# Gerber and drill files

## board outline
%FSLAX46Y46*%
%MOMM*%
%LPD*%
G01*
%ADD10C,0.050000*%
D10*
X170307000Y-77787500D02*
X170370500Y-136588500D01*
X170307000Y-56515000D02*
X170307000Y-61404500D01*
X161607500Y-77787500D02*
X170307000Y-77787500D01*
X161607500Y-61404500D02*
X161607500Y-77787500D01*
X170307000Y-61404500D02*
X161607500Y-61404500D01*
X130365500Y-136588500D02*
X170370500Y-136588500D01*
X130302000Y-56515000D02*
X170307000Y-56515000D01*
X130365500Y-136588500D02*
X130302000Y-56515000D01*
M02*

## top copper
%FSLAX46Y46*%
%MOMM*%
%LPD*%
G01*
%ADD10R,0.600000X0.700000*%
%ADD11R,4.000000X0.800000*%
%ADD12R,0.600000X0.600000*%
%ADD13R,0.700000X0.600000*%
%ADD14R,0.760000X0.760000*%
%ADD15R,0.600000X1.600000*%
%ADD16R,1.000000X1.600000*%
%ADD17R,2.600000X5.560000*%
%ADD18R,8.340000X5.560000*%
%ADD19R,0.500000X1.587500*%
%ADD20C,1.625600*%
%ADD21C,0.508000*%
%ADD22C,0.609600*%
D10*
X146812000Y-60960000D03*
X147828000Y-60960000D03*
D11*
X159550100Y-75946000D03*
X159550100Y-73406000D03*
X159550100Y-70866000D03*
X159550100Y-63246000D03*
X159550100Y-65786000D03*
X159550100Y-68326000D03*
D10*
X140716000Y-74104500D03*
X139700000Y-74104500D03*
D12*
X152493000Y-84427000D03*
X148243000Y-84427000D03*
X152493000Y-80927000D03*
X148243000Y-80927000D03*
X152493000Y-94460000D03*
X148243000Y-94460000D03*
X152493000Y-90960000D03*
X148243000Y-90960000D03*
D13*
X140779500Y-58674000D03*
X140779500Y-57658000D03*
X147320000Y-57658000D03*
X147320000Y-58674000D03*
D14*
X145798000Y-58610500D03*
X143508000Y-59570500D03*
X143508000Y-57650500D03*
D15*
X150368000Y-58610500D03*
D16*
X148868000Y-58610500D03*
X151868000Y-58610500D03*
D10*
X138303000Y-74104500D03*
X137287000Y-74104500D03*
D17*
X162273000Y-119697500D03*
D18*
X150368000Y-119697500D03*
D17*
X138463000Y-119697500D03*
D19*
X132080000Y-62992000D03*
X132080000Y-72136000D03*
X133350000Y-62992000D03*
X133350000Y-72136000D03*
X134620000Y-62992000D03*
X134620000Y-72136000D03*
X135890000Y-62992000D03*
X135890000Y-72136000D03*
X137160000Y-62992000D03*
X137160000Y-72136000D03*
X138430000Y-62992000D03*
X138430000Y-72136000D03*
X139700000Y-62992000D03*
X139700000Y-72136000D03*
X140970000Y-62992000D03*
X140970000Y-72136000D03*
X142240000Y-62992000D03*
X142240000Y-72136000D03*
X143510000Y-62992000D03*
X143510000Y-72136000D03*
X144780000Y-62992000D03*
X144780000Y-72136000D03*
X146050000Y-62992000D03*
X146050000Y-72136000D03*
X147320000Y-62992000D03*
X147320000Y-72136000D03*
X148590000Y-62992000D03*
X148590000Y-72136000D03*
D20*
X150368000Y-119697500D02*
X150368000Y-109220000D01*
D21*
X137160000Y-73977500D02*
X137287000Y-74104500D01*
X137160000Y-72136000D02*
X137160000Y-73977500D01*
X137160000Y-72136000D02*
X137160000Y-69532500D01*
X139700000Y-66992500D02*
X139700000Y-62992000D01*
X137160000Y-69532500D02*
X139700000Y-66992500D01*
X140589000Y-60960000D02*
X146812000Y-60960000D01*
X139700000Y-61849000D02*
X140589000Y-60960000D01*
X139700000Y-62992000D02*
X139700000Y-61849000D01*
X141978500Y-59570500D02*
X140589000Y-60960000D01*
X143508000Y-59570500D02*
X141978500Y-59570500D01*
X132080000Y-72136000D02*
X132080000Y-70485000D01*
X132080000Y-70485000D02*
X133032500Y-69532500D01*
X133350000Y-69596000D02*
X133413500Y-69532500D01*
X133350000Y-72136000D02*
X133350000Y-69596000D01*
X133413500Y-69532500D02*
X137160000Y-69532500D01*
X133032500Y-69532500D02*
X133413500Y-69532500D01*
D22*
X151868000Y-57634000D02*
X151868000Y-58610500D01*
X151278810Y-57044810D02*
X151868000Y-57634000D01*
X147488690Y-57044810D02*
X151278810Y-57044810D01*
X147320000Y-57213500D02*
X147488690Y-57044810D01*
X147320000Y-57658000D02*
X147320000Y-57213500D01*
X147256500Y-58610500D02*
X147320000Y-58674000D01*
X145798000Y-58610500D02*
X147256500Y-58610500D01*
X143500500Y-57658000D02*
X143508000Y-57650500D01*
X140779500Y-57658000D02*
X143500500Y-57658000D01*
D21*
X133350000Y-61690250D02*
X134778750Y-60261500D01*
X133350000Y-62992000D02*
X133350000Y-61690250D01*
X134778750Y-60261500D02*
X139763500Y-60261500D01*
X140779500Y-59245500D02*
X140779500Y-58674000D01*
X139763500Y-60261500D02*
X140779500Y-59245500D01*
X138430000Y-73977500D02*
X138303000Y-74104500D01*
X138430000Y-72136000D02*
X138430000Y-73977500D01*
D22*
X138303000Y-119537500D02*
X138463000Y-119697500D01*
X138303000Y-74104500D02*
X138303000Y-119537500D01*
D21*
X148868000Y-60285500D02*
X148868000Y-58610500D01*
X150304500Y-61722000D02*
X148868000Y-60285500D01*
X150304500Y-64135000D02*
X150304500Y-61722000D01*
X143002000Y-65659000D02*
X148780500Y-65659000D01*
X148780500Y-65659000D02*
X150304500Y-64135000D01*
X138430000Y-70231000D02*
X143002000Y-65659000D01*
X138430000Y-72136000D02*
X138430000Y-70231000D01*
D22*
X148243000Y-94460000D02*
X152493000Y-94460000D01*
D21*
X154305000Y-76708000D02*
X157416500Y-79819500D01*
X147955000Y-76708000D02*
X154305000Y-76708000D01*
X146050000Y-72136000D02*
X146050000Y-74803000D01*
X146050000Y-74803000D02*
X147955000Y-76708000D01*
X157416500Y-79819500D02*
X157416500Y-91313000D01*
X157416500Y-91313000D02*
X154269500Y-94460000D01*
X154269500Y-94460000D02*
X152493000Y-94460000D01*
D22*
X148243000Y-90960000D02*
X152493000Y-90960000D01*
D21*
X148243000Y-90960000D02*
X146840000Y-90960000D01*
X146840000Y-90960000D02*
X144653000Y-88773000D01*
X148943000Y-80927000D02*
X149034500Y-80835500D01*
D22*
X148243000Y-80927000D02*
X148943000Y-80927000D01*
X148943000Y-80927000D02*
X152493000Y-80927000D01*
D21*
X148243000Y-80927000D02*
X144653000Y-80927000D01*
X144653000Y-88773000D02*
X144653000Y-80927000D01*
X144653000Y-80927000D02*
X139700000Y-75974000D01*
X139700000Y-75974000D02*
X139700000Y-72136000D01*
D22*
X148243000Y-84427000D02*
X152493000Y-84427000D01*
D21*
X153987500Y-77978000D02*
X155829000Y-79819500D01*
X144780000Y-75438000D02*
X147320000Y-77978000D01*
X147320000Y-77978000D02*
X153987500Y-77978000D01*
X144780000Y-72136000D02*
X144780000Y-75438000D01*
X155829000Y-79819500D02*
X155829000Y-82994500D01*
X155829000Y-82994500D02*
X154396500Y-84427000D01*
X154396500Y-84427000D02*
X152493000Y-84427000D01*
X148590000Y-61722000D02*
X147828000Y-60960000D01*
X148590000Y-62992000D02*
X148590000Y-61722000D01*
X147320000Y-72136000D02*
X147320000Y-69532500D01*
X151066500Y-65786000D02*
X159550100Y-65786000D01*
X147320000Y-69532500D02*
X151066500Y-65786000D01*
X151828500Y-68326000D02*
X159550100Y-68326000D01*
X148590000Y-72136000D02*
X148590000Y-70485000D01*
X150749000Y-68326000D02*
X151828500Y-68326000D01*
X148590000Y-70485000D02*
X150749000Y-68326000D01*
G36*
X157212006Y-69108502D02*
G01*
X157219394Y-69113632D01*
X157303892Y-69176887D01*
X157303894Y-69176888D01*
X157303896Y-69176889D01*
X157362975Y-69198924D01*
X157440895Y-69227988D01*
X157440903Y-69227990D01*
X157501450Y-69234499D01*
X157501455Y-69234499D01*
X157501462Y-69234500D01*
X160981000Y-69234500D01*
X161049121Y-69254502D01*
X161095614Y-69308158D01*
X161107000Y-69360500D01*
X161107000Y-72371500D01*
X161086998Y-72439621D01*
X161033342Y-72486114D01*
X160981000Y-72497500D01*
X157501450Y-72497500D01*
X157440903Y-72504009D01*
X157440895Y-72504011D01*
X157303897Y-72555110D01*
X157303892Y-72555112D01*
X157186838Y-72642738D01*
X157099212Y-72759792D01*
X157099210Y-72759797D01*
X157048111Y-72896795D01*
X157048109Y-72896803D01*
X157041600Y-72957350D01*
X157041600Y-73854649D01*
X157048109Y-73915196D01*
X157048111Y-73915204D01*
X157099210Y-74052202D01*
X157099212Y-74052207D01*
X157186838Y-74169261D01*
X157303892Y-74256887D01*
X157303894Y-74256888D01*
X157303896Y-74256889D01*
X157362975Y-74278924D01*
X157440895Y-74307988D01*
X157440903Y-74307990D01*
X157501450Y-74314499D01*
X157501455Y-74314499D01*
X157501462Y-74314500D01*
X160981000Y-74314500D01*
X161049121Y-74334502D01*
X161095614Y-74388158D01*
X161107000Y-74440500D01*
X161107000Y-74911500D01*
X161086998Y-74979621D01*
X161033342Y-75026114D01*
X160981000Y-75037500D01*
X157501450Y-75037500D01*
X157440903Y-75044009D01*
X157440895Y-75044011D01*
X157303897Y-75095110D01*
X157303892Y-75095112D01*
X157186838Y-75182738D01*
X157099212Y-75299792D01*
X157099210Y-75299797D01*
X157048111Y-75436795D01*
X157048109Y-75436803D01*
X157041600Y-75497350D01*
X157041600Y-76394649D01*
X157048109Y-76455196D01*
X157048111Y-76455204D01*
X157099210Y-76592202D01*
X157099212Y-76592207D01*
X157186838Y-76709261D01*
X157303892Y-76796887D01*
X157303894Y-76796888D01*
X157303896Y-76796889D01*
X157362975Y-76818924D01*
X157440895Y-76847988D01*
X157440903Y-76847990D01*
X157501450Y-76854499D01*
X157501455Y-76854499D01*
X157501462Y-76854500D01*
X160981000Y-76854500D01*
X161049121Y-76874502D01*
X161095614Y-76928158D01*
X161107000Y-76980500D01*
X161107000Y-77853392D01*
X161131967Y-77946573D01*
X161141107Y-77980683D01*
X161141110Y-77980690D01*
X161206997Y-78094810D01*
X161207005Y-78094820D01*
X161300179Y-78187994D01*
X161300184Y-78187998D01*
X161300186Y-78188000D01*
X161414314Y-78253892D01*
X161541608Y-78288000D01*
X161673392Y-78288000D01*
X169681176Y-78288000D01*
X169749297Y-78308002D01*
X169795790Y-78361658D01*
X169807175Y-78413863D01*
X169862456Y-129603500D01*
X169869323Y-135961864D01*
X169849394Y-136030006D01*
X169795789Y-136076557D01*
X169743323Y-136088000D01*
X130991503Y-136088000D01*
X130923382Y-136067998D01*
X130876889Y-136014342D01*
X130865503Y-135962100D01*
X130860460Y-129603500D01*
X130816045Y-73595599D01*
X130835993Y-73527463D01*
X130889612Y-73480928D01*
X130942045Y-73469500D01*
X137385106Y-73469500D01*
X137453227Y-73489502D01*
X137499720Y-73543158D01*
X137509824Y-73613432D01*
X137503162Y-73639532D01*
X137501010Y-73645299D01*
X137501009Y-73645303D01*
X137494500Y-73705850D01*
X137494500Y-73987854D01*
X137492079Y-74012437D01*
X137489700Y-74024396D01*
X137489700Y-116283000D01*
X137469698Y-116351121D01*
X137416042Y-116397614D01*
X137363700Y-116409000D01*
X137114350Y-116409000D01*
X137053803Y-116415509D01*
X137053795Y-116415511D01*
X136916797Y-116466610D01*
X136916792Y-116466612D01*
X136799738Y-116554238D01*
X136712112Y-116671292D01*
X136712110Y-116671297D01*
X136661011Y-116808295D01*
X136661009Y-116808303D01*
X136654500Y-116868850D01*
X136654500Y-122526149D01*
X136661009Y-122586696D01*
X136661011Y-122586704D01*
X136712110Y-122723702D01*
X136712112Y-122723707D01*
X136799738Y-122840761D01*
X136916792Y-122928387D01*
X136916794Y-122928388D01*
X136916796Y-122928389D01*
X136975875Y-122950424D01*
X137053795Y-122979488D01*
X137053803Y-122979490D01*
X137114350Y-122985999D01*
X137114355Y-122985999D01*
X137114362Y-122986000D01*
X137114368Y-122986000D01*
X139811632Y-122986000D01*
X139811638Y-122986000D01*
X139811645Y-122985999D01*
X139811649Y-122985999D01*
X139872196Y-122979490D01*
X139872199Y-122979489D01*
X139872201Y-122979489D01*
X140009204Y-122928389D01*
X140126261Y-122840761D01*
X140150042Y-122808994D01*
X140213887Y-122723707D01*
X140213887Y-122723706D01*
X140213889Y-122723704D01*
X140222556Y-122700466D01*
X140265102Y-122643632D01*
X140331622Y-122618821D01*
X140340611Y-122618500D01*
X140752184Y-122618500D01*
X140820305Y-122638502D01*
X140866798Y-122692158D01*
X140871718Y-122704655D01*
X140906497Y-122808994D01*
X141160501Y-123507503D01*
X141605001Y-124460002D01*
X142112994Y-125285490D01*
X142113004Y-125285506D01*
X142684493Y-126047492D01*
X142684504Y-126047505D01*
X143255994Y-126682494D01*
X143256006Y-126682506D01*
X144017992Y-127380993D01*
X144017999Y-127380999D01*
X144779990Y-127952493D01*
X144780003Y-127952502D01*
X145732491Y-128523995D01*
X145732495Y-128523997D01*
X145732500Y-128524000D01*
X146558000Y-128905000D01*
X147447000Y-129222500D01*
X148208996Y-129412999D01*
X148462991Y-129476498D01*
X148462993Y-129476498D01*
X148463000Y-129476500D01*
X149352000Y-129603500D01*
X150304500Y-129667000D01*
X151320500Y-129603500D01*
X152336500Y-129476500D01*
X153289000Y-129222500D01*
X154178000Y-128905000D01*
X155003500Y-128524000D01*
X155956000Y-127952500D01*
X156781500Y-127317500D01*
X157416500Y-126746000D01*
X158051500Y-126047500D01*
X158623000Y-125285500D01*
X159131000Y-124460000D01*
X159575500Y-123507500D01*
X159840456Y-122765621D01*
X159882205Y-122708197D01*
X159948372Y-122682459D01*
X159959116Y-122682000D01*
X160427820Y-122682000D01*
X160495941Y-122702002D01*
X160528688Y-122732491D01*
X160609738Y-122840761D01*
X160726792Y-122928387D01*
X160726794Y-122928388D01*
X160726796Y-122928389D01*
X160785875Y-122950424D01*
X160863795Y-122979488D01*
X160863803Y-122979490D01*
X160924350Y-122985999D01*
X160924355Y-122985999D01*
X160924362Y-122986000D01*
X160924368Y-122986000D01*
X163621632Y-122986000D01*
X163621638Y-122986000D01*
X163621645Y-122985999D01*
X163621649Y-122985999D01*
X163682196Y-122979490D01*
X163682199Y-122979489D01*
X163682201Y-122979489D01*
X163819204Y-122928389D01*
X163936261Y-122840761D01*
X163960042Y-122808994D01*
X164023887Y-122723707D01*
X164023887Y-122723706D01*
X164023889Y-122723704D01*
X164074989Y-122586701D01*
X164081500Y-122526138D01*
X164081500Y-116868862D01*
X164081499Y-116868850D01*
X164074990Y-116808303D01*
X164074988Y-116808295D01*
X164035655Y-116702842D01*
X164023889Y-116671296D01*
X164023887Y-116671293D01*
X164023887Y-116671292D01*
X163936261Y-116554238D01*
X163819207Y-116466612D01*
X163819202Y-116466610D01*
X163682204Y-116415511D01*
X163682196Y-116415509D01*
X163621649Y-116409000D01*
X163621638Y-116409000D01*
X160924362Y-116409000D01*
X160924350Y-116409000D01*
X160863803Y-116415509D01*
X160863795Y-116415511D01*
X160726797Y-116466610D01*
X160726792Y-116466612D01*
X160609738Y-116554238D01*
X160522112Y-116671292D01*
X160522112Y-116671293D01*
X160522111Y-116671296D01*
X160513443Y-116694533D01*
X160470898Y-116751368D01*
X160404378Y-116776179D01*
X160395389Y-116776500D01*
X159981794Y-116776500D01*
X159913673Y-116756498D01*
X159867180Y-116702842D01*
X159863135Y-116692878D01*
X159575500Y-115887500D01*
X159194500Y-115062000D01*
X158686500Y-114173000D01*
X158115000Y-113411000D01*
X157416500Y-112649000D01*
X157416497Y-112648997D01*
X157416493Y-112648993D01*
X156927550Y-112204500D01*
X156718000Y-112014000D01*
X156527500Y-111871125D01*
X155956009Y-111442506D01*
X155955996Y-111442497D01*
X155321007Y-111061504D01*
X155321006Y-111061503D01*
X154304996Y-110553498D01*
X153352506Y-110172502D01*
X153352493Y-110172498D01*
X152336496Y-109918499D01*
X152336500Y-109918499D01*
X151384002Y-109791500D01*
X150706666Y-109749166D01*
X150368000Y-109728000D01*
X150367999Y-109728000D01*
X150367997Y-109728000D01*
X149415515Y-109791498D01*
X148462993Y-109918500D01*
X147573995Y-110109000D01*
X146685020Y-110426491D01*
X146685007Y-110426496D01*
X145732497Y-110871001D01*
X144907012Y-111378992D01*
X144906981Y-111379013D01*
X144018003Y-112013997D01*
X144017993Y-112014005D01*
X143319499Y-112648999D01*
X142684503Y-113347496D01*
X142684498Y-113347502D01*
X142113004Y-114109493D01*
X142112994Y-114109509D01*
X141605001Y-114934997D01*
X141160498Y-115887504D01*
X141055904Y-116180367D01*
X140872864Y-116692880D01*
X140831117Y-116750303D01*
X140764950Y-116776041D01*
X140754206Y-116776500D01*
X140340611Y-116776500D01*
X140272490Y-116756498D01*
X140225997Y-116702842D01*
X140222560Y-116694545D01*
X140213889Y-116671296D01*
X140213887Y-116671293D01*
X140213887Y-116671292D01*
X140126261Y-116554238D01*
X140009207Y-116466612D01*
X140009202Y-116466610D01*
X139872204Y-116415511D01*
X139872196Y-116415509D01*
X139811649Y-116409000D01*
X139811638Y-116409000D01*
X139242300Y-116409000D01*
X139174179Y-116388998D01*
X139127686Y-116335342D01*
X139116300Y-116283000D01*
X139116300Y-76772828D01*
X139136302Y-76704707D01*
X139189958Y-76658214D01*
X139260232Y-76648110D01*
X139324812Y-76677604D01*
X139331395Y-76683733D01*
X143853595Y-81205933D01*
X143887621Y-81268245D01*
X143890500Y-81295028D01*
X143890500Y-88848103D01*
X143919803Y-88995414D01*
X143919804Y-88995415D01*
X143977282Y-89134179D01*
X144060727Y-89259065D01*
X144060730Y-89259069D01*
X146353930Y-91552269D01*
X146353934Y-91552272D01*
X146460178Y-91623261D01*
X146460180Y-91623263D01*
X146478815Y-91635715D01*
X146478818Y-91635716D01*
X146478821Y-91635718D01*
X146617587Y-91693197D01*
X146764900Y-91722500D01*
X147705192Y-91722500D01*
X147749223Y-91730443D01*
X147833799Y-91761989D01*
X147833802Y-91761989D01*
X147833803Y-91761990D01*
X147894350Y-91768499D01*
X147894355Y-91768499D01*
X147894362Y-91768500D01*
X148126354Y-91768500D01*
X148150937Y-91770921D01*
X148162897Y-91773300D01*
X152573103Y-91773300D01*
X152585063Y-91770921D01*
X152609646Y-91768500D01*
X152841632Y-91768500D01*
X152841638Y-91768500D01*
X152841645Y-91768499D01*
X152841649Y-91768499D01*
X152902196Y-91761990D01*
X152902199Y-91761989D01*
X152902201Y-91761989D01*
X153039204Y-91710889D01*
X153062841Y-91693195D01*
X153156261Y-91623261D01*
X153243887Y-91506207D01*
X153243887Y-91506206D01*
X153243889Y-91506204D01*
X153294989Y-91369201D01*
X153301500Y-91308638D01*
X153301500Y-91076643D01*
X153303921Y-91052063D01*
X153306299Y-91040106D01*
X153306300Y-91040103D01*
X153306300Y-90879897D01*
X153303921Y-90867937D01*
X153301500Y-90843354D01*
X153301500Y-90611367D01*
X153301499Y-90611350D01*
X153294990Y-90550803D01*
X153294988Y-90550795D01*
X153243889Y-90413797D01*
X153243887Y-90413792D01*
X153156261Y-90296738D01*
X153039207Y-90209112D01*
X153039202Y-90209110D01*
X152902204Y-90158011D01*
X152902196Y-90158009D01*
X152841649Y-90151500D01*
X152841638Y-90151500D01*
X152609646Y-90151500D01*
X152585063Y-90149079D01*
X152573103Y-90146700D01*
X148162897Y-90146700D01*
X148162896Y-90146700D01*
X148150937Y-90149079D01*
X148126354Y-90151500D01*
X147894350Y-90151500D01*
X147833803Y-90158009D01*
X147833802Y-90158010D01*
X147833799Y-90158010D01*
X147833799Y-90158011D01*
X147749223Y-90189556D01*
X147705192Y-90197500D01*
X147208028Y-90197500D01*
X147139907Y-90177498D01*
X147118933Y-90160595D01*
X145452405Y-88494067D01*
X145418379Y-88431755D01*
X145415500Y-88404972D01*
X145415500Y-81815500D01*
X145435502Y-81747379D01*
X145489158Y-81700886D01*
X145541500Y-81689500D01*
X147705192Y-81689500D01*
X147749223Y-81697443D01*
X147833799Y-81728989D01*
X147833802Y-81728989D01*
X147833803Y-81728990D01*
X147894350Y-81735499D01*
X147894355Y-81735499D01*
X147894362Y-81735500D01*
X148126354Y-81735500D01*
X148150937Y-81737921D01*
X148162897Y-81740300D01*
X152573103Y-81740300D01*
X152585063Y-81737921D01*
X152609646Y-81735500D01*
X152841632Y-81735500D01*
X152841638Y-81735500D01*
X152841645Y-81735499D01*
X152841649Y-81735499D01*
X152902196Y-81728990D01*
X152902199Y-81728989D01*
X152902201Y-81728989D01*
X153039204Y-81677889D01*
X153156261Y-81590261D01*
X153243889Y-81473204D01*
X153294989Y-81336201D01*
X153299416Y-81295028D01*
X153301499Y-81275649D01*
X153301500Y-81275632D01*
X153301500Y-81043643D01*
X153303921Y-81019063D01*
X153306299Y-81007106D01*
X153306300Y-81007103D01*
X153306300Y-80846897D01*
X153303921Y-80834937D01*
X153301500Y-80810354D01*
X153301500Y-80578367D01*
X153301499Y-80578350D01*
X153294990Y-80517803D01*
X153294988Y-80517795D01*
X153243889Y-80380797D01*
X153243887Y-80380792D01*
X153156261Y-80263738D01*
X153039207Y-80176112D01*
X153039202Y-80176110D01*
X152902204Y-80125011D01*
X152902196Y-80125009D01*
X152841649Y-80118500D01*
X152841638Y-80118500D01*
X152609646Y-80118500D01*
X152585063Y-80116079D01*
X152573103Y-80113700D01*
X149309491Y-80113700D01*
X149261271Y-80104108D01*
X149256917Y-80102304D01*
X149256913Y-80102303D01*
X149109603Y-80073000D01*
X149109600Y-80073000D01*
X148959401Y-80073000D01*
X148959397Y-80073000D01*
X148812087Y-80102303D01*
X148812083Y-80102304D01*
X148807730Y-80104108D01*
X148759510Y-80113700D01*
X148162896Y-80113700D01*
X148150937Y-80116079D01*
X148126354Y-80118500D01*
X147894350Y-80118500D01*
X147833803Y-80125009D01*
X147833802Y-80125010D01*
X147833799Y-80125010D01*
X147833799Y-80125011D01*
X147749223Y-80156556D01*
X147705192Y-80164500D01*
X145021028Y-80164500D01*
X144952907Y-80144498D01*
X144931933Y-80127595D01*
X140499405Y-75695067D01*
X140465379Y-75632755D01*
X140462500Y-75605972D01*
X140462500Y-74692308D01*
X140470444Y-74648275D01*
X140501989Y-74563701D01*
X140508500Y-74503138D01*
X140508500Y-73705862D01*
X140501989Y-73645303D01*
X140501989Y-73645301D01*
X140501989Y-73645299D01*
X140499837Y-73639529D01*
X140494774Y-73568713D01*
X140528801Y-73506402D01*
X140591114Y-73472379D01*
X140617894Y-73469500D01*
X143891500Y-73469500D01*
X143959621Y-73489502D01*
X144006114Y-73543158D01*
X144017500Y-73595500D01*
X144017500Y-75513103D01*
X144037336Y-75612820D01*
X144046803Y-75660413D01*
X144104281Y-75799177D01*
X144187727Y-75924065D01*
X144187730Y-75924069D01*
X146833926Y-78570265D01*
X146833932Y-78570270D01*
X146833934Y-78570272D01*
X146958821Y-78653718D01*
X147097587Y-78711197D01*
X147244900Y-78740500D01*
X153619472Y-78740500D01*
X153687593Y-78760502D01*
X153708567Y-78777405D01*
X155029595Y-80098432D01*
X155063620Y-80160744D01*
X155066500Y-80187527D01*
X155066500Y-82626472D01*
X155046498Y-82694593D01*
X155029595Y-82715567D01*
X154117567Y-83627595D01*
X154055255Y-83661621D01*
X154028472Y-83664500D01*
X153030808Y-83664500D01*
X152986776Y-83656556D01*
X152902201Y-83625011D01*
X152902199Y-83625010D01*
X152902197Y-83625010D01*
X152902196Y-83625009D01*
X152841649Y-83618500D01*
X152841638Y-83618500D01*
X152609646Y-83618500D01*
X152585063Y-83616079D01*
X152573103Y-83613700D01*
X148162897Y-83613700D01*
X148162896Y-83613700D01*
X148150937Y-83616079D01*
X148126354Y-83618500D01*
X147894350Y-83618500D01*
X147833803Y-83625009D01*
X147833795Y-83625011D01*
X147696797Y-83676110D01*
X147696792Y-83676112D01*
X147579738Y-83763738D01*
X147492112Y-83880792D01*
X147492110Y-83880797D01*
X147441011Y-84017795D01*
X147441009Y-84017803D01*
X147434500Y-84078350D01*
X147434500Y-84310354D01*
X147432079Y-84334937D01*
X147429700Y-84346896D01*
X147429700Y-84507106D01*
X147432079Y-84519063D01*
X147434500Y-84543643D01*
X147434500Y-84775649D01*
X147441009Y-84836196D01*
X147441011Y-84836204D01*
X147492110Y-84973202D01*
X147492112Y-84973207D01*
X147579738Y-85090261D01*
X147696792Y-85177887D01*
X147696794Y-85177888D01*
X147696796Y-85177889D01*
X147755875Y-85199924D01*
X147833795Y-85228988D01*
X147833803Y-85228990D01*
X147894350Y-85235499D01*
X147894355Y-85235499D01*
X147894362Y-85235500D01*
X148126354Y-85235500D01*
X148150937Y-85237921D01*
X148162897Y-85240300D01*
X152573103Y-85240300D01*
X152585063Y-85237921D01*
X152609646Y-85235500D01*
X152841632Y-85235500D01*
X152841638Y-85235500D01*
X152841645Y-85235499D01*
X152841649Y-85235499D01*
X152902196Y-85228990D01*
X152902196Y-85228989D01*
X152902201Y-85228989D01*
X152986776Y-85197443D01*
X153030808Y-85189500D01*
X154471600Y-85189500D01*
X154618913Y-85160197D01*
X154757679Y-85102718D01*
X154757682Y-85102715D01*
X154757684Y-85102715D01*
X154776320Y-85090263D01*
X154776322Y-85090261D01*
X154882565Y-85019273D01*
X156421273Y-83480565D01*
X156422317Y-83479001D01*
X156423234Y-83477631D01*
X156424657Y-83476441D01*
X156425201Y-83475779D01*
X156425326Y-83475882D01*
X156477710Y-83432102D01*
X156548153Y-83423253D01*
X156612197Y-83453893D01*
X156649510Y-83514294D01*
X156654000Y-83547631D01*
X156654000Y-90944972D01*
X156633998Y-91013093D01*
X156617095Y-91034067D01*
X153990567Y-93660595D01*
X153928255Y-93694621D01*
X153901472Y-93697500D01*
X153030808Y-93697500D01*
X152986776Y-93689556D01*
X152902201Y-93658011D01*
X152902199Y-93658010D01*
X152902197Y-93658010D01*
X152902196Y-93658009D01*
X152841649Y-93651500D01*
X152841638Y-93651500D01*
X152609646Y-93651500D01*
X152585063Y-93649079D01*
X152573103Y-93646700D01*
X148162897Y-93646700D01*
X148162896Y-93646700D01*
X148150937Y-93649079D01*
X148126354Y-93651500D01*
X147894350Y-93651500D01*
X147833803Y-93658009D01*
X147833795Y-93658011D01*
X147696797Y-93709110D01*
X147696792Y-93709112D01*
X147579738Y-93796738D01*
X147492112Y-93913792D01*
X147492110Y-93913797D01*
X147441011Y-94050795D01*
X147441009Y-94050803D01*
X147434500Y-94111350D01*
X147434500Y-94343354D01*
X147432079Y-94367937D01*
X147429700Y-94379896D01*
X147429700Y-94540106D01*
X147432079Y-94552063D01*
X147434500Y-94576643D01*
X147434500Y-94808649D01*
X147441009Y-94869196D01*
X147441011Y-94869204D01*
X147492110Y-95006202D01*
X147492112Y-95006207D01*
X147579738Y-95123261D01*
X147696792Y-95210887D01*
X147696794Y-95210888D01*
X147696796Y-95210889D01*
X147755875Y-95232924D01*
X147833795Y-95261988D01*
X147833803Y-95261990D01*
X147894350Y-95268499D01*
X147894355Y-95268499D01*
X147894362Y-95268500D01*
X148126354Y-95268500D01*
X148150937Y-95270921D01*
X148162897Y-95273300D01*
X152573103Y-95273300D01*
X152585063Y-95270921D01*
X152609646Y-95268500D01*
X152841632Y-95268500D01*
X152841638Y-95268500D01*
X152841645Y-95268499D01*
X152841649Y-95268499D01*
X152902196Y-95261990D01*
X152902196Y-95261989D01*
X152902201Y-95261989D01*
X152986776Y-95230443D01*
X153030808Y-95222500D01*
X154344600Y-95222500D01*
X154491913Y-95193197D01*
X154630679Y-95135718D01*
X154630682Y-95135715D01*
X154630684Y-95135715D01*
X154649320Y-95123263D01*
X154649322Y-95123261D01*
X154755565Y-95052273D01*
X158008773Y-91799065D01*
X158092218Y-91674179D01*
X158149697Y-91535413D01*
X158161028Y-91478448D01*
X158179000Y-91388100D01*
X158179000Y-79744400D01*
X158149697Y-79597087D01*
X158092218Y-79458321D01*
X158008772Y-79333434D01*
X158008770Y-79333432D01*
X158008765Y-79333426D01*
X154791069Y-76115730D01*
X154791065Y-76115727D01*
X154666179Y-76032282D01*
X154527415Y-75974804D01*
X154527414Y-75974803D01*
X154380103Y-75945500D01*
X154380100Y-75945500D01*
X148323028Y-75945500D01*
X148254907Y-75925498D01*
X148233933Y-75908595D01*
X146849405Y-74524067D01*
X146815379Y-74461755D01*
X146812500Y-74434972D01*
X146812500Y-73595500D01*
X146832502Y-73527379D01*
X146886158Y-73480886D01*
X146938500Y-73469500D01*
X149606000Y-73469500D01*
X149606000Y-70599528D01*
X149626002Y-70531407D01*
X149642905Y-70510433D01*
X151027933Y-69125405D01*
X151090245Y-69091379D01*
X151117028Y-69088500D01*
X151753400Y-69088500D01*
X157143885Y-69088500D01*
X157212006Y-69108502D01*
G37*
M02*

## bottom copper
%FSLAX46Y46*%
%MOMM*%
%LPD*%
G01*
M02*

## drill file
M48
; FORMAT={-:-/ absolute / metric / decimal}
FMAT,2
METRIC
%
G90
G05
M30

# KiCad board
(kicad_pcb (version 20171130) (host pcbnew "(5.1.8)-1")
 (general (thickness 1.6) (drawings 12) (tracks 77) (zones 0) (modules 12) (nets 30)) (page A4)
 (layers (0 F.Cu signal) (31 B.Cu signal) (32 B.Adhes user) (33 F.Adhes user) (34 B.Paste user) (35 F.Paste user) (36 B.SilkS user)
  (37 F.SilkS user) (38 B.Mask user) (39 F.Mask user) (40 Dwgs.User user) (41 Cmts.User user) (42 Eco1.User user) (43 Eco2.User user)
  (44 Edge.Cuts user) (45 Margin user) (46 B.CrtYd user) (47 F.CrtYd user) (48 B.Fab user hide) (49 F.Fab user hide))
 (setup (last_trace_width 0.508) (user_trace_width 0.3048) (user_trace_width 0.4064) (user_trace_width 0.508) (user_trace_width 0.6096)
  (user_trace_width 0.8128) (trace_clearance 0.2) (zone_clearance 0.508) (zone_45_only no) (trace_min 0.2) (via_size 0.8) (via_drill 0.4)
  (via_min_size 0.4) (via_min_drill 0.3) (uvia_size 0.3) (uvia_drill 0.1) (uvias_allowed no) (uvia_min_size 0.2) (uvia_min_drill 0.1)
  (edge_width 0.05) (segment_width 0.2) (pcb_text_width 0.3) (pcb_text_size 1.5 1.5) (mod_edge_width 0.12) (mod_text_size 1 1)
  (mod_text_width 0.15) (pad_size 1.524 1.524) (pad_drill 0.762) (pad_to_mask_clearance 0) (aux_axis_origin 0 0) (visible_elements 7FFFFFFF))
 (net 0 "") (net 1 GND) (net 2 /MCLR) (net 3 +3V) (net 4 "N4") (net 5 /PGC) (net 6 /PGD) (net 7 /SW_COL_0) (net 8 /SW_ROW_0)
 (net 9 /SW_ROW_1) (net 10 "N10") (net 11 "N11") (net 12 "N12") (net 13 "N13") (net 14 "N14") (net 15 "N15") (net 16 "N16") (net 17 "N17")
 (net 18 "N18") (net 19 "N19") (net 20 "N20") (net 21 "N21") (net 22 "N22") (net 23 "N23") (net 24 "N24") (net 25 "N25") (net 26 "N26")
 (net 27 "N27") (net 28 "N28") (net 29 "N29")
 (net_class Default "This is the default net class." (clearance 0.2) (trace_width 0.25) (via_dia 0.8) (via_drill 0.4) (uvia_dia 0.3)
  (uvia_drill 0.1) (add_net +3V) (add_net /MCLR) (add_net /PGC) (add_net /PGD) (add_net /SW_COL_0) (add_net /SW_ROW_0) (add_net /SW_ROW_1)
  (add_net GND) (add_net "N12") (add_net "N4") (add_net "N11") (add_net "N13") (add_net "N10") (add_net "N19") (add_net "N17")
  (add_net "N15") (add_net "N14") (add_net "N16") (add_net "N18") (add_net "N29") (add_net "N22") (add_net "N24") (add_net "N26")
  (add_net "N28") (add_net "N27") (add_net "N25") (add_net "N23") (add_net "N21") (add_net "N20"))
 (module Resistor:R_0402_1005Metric (layer F.Cu) (at 147.32 60.96 180)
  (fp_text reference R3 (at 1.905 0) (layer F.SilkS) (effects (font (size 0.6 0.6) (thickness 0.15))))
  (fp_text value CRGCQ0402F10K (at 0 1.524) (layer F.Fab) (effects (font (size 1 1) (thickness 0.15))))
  (pad 2 smd rect (at 0.508 0 180) (size 0.6 0.7) (layers F.Cu F.Paste F.Mask) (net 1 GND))
  (pad 1 smd rect (at -0.508 0 180) (size 0.6 0.7) (layers F.Cu F.Paste F.Mask) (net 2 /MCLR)))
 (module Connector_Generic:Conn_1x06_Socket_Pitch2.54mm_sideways (layer F.Cu) (at 166.0525 69.596 270)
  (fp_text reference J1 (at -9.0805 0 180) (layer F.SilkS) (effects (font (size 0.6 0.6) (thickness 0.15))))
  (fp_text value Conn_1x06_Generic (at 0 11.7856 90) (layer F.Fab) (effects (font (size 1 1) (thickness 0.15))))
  (pad 6 smd rect (at 6.35 6.5024 270) (size 0.8 4) (layers F.Cu F.Paste F.Mask) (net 2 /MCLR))
  (pad 5 smd rect (at 3.81 6.5024 270) (size 0.8 4) (layers F.Cu F.Paste F.Mask) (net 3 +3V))
  (pad 4 smd rect (at 1.27 6.5024 270) (size 0.8 4) (layers F.Cu F.Paste F.Mask) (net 1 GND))
  (pad 1 smd rect (at -6.35 6.5024 270) (size 0.8 4) (layers F.Cu F.Paste F.Mask) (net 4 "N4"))
  (pad 2 smd rect (at -3.81 6.5024 270) (size 0.8 4) (layers F.Cu F.Paste F.Mask) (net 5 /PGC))
  (pad 3 smd rect (at -1.27 6.5024 270) (size 0.8 4) (layers F.Cu F.Paste F.Mask) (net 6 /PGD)))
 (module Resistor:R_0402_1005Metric (layer F.Cu) (at 140.208 74.1045)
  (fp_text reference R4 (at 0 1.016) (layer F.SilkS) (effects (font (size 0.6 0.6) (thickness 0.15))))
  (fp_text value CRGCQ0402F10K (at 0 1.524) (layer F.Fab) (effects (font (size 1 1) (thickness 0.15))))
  (pad 2 smd rect (at 0.508 0) (size 0.6 0.7) (layers F.Cu F.Paste F.Mask) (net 1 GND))
  (pad 1 smd rect (at -0.508 0) (size 0.6 0.7) (layers F.Cu F.Paste F.Mask) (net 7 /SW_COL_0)))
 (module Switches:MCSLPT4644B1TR (layer F.Cu) (at 150.368 82.677)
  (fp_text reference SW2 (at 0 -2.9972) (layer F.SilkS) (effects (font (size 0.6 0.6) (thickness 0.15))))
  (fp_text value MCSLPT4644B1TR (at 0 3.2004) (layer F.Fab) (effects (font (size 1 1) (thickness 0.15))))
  (pad 2 smd rect (at 2.125 1.75) (size 0.6 0.6) (layers F.Cu F.Paste F.Mask) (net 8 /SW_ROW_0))
  (pad 2 smd rect (at -2.125 1.75) (size 0.6 0.6) (layers F.Cu F.Paste F.Mask) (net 8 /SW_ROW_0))
  (pad 1 smd rect (at 2.125 -1.75) (size 0.6 0.6) (layers F.Cu F.Paste F.Mask) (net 7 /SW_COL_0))
  (pad 1 smd rect (at -2.125 -1.75) (size 0.6 0.6) (layers F.Cu F.Paste F.Mask) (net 7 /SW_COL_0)))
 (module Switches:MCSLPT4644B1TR (layer F.Cu) (at 150.368 92.71)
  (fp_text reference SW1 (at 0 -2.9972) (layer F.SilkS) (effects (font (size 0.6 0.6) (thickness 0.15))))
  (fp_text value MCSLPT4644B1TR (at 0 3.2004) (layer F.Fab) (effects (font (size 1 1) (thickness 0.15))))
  (pad 2 smd rect (at 2.125 1.75) (size 0.6 0.6) (layers F.Cu F.Paste F.Mask) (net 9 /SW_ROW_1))
  (pad 2 smd rect (at -2.125 1.75) (size 0.6 0.6) (layers F.Cu F.Paste F.Mask) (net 9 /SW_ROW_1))
  (pad 1 smd rect (at 2.125 -1.75) (size 0.6 0.6) (layers F.Cu F.Paste F.Mask) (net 7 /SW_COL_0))
  (pad 1 smd rect (at -2.125 -1.75) (size 0.6 0.6) (layers F.Cu F.Paste F.Mask) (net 7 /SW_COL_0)))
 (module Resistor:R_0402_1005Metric (layer F.Cu) (at 140.7795 58.166 270)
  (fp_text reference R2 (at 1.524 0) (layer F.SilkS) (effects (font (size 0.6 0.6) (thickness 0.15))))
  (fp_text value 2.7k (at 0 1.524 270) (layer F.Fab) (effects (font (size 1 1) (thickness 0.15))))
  (pad 2 smd rect (at 0.508 0 270) (size 0.6 0.7) (layers F.Cu F.Paste F.Mask) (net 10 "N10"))
  (pad 1 smd rect (at -0.508 0 270) (size 0.6 0.7) (layers F.Cu F.Paste F.Mask) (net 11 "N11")))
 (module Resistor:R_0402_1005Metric (layer F.Cu) (at 147.32 58.166 90)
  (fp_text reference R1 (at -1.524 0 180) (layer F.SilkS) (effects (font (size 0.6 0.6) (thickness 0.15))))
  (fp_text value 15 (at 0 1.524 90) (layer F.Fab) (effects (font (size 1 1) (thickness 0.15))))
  (pad 2 smd rect (at 0.508 0 90) (size 0.6 0.7) (layers F.Cu F.Paste F.Mask) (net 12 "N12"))
  (pad 1 smd rect (at -0.508 0 90) (size 0.6 0.7) (layers F.Cu F.Paste F.Mask) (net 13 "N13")))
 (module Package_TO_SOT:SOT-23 (layer F.Cu) (at 144.653 58.6105)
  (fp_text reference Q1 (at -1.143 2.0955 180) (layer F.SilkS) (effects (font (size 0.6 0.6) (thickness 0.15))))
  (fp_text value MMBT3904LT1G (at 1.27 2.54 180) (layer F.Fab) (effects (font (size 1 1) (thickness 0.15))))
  (pad 3 smd rect (at 1.145 0 270) (size 0.76 0.76) (layers F.Cu F.Paste F.Mask) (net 13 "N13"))
  (pad 2 smd rect (at -1.145 0.96 90) (size 0.76 0.76) (layers F.Cu F.Paste F.Mask) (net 1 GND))
  (pad 1 smd rect (at -1.145 -0.96 90) (size 0.76 0.76) (layers F.Cu F.Paste F.Mask) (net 11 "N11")))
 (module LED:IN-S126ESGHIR (layer F.Cu) (at 150.368 58.6105 180)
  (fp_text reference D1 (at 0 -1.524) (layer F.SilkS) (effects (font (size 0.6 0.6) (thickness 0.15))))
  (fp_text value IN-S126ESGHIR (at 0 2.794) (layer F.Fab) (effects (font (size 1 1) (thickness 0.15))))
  (pad "" smd rect (at 0 0 180) (size 0.6 1.6) (layers F.Cu F.Paste F.Mask))
  (pad 2 smd rect (at 1.5 0 180) (size 1 1.6) (layers F.Cu F.Paste F.Mask) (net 3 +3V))
  (pad 1 smd rect (at -1.5 0 180) (size 1 1.6) (layers F.Cu F.Paste F.Mask) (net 12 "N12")))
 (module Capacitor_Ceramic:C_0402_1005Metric (layer F.Cu) (at 137.795 74.1045)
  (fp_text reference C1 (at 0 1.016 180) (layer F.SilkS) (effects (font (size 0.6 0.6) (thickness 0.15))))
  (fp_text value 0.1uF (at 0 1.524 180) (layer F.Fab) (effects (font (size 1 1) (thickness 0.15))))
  (pad 2 smd rect (at 0.508 0) (size 0.6 0.7) (layers F.Cu F.Paste F.Mask) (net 3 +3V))
  (pad 1 smd rect (at -0.508 0) (size 0.6 0.7) (layers F.Cu F.Paste F.Mask) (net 1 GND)))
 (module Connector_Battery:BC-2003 (layer F.Cu) (at 150.368 119.6975)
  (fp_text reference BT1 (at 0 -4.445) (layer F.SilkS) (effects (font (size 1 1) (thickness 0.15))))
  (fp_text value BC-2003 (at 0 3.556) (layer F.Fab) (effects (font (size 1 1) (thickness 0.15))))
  (pad 1 smd rect (at 11.905 0) (size 2.6 5.56) (layers F.Cu F.Paste F.Mask) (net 3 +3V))
  (pad 2 smd rect (at 0 0) (size 8.34 5.56) (layers F.Cu F.Paste F.Mask) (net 1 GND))
  (pad 1 smd rect (at -11.905 0) (size 2.6 5.56) (layers F.Cu F.Paste F.Mask) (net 3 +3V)))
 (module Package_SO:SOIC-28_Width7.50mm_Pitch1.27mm (layer F.Cu) (at 140.335 67.564 270)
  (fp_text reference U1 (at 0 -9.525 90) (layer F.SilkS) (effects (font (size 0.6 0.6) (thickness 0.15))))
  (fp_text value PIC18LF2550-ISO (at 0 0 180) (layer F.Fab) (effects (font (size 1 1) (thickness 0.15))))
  (pad 14 smd rect (at -4.572 8.255 180) (size 0.5 1.5875) (layers F.Cu F.Paste F.Mask) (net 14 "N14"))
  (pad 15 smd rect (at 4.572 8.255 180) (size 0.5 1.5875) (layers F.Cu F.Paste F.Mask) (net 1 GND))
  (pad 13 smd rect (at -4.572 6.985 180) (size 0.5 1.5875) (layers F.Cu F.Paste F.Mask) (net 10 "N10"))
  (pad 16 smd rect (at 4.572 6.985 180) (size 0.5 1.5875) (layers F.Cu F.Paste F.Mask) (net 1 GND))
  (pad 12 smd rect (at -4.572 5.715 180) (size 0.5 1.5875) (layers F.Cu F.Paste F.Mask) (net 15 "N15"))
  (pad 17 smd rect (at 4.572 5.715 180) (size 0.5 1.5875) (layers F.Cu F.Paste F.Mask) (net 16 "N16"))
  (pad 11 smd rect (at -4.572 4.445 180) (size 0.5 1.5875) (layers F.Cu F.Paste F.Mask) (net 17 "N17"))
  (pad 18 smd rect (at 4.572 4.445 180) (size 0.5 1.5875) (layers F.Cu F.Paste F.Mask) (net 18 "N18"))
  (pad 10 smd rect (at -4.572 3.175 180) (size 0.5 1.5875) (layers F.Cu F.Paste F.Mask) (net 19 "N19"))
  (pad 19 smd rect (at 4.572 3.175 180) (size 0.5 1.5875) (layers F.Cu F.Paste F.Mask) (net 1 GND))
  (pad 9 smd rect (at -4.572 1.905 180) (size 0.5 1.5875) (layers F.Cu F.Paste F.Mask) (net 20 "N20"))
  (pad 20 smd rect (at 4.572 1.905 180) (size 0.5 1.5875) (layers F.Cu F.Paste F.Mask) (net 3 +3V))
  (pad 8 smd rect (at -4.572 0.635 180) (size 0.5 1.5875) (layers F.Cu F.Paste F.Mask) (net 1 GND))
  (pad 21 smd rect (at 4.572 0.635 180) (size 0.5 1.5875) (layers F.Cu F.Paste F.Mask) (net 7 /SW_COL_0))
  (pad 7 smd rect (at -4.572 -0.635 180) (size 0.5 1.5875) (layers F.Cu F.Paste F.Mask) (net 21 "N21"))
  (pad 22 smd rect (at 4.572 -0.635 180) (size 0.5 1.5875) (layers F.Cu F.Paste F.Mask) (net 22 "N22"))
  (pad 6 smd rect (at -4.572 -1.905 180) (size 0.5 1.5875) (layers F.Cu F.Paste F.Mask) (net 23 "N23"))
  (pad 23 smd rect (at 4.572 -1.905 180) (size 0.5 1.5875) (layers F.Cu F.Paste F.Mask) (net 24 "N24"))
  (pad 5 smd rect (at -4.572 -3.175 180) (size 0.5 1.5875) (layers F.Cu F.Paste F.Mask) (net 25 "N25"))
  (pad 24 smd rect (at 4.572 -3.175 180) (size 0.5 1.5875) (layers F.Cu F.Paste F.Mask) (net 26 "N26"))
  (pad 4 smd rect (at -4.572 -4.445 180) (size 0.5 1.5875) (layers F.Cu F.Paste F.Mask) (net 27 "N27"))
  (pad 25 smd rect (at 4.572 -4.445 180) (size 0.5 1.5875) (layers F.Cu F.Paste F.Mask) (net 8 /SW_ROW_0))
  (pad 3 smd rect (at -4.572 -5.715 180) (size 0.5 1.5875) (layers F.Cu F.Paste F.Mask) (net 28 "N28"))
  (pad 26 smd rect (at 4.572 -5.715 180) (size 0.5 1.5875) (layers F.Cu F.Paste F.Mask) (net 9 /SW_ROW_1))
  (pad 2 smd rect (at -4.572 -6.985 180) (size 0.5 1.5875) (layers F.Cu F.Paste F.Mask) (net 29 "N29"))
  (pad 27 smd rect (at 4.572 -6.985 180) (size 0.5 1.5875) (layers F.Cu F.Paste F.Mask) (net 5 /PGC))
  (pad 1 smd rect (at -4.572 -8.255 180) (size 0.5 1.5875) (layers F.Cu F.Paste F.Mask) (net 2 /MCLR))
  (pad 28 smd rect (at 4.572 -8.255 180) (size 0.5 1.5875) (layers F.Cu F.Paste F.Mask) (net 6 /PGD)))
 (gr_line (start 170.307 77.7875) (end 170.3705 136.5885) (layer Edge.Cuts) (width 0.05))
 (gr_line (start 170.307 56.515) (end 170.307 61.4045) (layer Edge.Cuts) (width 0.05))
 (gr_line (start 161.6075 77.7875) (end 170.307 77.7875) (layer Edge.Cuts) (width 0.05))
 (gr_line (start 161.6075 61.4045) (end 161.6075 77.7875) (layer Edge.Cuts) (width 0.05))
 (gr_line (start 170.307 61.4045) (end 161.6075 61.4045) (layer Edge.Cuts) (width 0.05))
 (gr_line (start 130.3655 136.5885) (end 170.3705 136.5885) (layer Edge.Cuts) (width 0.05))
 (gr_line (start 130.302 56.515) (end 170.307 56.515) (layer Edge.Cuts) (width 0.05))
 (gr_line (start 130.3655 136.5885) (end 130.302 56.515) (layer Edge.Cuts) (width 0.05))
 (segment (start 150.368 119.6975) (end 150.368 109.22) (width 1.6256) (layer F.Cu) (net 1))
 (segment (start 137.16 73.9775) (end 137.287 74.1045) (width 0.508) (layer F.Cu) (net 1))
 (segment (start 137.16 72.136) (end 137.16 73.9775) (width 0.508) (layer F.Cu) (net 1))
 (segment (start 137.16 72.136) (end 137.16 69.5325) (width 0.508) (layer F.Cu) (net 1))
 (segment (start 139.7 66.9925) (end 139.7 62.992) (width 0.508) (layer F.Cu) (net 1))
 (segment (start 137.16 69.5325) (end 139.7 66.9925) (width 0.508) (layer F.Cu) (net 1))
 (segment (start 140.589 60.96) (end 146.812 60.96) (width 0.508) (layer F.Cu) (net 1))
 (segment (start 139.7 61.849) (end 140.589 60.96) (width 0.508) (layer F.Cu) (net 1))
 (segment (start 139.7 62.992) (end 139.7 61.849) (width 0.508) (layer F.Cu) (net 1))
 (segment (start 141.9785 59.5705) (end 140.589 60.96) (width 0.508) (layer F.Cu) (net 1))
 (segment (start 143.508 59.5705) (end 141.9785 59.5705) (width 0.508) (layer F.Cu) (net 1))
 (segment (start 132.08 72.136) (end 132.08 70.485) (width 0.508) (layer F.Cu) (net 1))
 (segment (start 132.08 70.485) (end 133.0325 69.5325) (width 0.508) (layer F.Cu) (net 1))
 (segment (start 133.35 69.596) (end 133.4135 69.5325) (width 0.508) (layer F.Cu) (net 1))
 (segment (start 133.35 72.136) (end 133.35 69.596) (width 0.508) (layer F.Cu) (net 1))
 (segment (start 133.4135 69.5325) (end 137.16 69.5325) (width 0.508) (layer F.Cu) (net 1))
 (segment (start 133.0325 69.5325) (end 133.4135 69.5325) (width 0.508) (layer F.Cu) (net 1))
 (segment (start 151.868 57.634) (end 151.868 58.6105) (width 0.6096) (layer F.Cu) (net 12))
 (segment (start 151.27881 57.04481) (end 151.868 57.634) (width 0.6096) (layer F.Cu) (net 12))
 (segment (start 147.48869 57.04481) (end 151.27881 57.04481) (width 0.6096) (layer F.Cu) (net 12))
 (segment (start 147.32 57.2135) (end 147.48869 57.04481) (width 0.6096) (layer F.Cu) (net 12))
 (segment (start 147.32 57.658) (end 147.32 57.2135) (width 0.6096) (layer F.Cu) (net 12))
 (segment (start 147.2565 58.6105) (end 147.32 58.674) (width 0.6096) (layer F.Cu) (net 13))
 (segment (start 145.798 58.6105) (end 147.2565 58.6105) (width 0.6096) (layer F.Cu) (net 13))
 (segment (start 143.5005 57.658) (end 143.508 57.6505) (width 0.6096) (layer F.Cu) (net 11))
 (segment (start 140.7795 57.658) (end 143.5005 57.658) (width 0.6096) (layer F.Cu) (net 11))
 (segment (start 133.35 61.69025) (end 134.77875 60.2615) (width 0.508) (layer F.Cu) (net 10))
 (segment (start 133.35 62.992) (end 133.35 61.69025) (width 0.508) (layer F.Cu) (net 10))
 (segment (start 134.77875 60.2615) (end 139.7635 60.2615) (width 0.508) (layer F.Cu) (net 10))
 (segment (start 140.7795 59.2455) (end 140.7795 58.674) (width 0.508) (layer F.Cu) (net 10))
 (segment (start 139.7635 60.2615) (end 140.7795 59.2455) (width 0.508) (layer F.Cu) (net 10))
 (segment (start 138.43 73.9775) (end 138.303 74.1045) (width 0.508) (layer F.Cu) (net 3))
 (segment (start 138.43 72.136) (end 138.43 73.9775) (width 0.508) (layer F.Cu) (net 3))
 (segment (start 138.303 119.5375) (end 138.463 119.6975) (width 0.6096) (layer F.Cu) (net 3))
 (segment (start 138.303 74.1045) (end 138.303 119.5375) (width 0.6096) (layer F.Cu) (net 3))
 (segment (start 148.868 60.2855) (end 148.868 58.6105) (width 0.508) (layer F.Cu) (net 3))
 (segment (start 150.3045 61.722) (end 148.868 60.2855) (width 0.508) (layer F.Cu) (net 3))
 (segment (start 150.3045 64.135) (end 150.3045 61.722) (width 0.508) (layer F.Cu) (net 3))
 (segment (start 143.002 65.659) (end 148.7805 65.659) (width 0.508) (layer F.Cu) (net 3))
 (segment (start 148.7805 65.659) (end 150.3045 64.135) (width 0.508) (layer F.Cu) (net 3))
 (segment (start 138.43 70.231) (end 143.002 65.659) (width 0.508) (layer F.Cu) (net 3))
 (segment (start 138.43 72.136) (end 138.43 70.231) (width 0.508) (layer F.Cu) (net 3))
 (segment (start 148.243 94.46) (end 152.493 94.46) (width 0.6096) (layer F.Cu) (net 9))
 (segment (start 154.305 76.708) (end 157.4165 79.8195) (width 0.508) (layer F.Cu) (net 9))
 (segment (start 147.955 76.708) (end 154.305 76.708) (width 0.508) (layer F.Cu) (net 9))
 (segment (start 146.05 72.136) (end 146.05 74.803) (width 0.508) (layer F.Cu) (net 9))
 (segment (start 146.05 74.803) (end 147.955 76.708) (width 0.508) (layer F.Cu) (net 9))
 (segment (start 157.4165 79.8195) (end 157.4165 91.313) (width 0.508) (layer F.Cu) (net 9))
 (segment (start 157.4165 91.313) (end 154.2695 94.46) (width 0.508) (layer F.Cu) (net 9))
 (segment (start 154.2695 94.46) (end 152.493 94.46) (width 0.508) (layer F.Cu) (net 9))
 (segment (start 148.243 90.96) (end 152.493 90.96) (width 0.6096) (layer F.Cu) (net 7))
 (segment (start 148.243 90.96) (end 146.84 90.96) (width 0.508) (layer F.Cu) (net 7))
 (segment (start 146.84 90.96) (end 144.653 88.773) (width 0.508) (layer F.Cu) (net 7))
 (segment (start 148.943 80.927) (end 149.0345 80.8355) (width 0.508) (layer F.Cu) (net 7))
 (segment (start 148.243 80.927) (end 148.943 80.927) (width 0.6096) (layer F.Cu) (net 7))
 (segment (start 148.943 80.927) (end 152.493 80.927) (width 0.6096) (layer F.Cu) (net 7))
 (segment (start 148.243 80.927) (end 144.653 80.927) (width 0.508) (layer F.Cu) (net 7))
 (segment (start 144.653 88.773) (end 144.653 80.927) (width 0.508) (layer F.Cu) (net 7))
 (segment (start 144.653 80.927) (end 139.7 75.974) (width 0.508) (layer F.Cu) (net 7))
 (segment (start 139.7 75.974) (end 139.7 72.136) (width 0.508) (layer F.Cu) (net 7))
 (segment (start 148.243 84.427) (end 152.493 84.427) (width 0.6096) (layer F.Cu) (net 8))
 (segment (start 153.9875 77.978) (end 155.829 79.8195) (width 0.508) (layer F.Cu) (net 8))
 (segment (start 144.78 75.438) (end 147.32 77.978) (width 0.508) (layer F.Cu) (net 8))
 (segment (start 147.32 77.978) (end 153.9875 77.978) (width 0.508) (layer F.Cu) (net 8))
 (segment (start 144.78 72.136) (end 144.78 75.438) (width 0.508) (layer F.Cu) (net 8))
 (segment (start 155.829 79.8195) (end 155.829 82.9945) (width 0.508) (layer F.Cu) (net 8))
 (segment (start 155.829 82.9945) (end 154.3965 84.427) (width 0.508) (layer F.Cu) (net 8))
 (segment (start 154.3965 84.427) (end 152.493 84.427) (width 0.508) (layer F.Cu) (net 8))
 (segment (start 148.59 61.722) (end 147.828 60.96) (width 0.508) (layer F.Cu) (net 2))
 (segment (start 148.59 62.992) (end 148.59 61.722) (width 0.508) (layer F.Cu) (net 2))
 (segment (start 147.32 72.136) (end 147.32 69.5325) (width 0.508) (layer F.Cu) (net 5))
 (segment (start 151.0665 65.786) (end 159.5501 65.786) (width 0.508) (layer F.Cu) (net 5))
 (segment (start 147.32 69.5325) (end 151.0665 65.786) (width 0.508) (layer F.Cu) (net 5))
 (segment (start 151.8285 68.326) (end 159.5501 68.326) (width 0.508) (layer F.Cu) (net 6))
 (segment (start 148.59 72.136) (end 148.59 70.485) (width 0.508) (layer F.Cu) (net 6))
 (segment (start 150.749 68.326) (end 151.8285 68.326) (width 0.508) (layer F.Cu) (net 6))
 (segment (start 148.59 70.485) (end 150.749 68.326) (width 0.508) (layer F.Cu) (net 6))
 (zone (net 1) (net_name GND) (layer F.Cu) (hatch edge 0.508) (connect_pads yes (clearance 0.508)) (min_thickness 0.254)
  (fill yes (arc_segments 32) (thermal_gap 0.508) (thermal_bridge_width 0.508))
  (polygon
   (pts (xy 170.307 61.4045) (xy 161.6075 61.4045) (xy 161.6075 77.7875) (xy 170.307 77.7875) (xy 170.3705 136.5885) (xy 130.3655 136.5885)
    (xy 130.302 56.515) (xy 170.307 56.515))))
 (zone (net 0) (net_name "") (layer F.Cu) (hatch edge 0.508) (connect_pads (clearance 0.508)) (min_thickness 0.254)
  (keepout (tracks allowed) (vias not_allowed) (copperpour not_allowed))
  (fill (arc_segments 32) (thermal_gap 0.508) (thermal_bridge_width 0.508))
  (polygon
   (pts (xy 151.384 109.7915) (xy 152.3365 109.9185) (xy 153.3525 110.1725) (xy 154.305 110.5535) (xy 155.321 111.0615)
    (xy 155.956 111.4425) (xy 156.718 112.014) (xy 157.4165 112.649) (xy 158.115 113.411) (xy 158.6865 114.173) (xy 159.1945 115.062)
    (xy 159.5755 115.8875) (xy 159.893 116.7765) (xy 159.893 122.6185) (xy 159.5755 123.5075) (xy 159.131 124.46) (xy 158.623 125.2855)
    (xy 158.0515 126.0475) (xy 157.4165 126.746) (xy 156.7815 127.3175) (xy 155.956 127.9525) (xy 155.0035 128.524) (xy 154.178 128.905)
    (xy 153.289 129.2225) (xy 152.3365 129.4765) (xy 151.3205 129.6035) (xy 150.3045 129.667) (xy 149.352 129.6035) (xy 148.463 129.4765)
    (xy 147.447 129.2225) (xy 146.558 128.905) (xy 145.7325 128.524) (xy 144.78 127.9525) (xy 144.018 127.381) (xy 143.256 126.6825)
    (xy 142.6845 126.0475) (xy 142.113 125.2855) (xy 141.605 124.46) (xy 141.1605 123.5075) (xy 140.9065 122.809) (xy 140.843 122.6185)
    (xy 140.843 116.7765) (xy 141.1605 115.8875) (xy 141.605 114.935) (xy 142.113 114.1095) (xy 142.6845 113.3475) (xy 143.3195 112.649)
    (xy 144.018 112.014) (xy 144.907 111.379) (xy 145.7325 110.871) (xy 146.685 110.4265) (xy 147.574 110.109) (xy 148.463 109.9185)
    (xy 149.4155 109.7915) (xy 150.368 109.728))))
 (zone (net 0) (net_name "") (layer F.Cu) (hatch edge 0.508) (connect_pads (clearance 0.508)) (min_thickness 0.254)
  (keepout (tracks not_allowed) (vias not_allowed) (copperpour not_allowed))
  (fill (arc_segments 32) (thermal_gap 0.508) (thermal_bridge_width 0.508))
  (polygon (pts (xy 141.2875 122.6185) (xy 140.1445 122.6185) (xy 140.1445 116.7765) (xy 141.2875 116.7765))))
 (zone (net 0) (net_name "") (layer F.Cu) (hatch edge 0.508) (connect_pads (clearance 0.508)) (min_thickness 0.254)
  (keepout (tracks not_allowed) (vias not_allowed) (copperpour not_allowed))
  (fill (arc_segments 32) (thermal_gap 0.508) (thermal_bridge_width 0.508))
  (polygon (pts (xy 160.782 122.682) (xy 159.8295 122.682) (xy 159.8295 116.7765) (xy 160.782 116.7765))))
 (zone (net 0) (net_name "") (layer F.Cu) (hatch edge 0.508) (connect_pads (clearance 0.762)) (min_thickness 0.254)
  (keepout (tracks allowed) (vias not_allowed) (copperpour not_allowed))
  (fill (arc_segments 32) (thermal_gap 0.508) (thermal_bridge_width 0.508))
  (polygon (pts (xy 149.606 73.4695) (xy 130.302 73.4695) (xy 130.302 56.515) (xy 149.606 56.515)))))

